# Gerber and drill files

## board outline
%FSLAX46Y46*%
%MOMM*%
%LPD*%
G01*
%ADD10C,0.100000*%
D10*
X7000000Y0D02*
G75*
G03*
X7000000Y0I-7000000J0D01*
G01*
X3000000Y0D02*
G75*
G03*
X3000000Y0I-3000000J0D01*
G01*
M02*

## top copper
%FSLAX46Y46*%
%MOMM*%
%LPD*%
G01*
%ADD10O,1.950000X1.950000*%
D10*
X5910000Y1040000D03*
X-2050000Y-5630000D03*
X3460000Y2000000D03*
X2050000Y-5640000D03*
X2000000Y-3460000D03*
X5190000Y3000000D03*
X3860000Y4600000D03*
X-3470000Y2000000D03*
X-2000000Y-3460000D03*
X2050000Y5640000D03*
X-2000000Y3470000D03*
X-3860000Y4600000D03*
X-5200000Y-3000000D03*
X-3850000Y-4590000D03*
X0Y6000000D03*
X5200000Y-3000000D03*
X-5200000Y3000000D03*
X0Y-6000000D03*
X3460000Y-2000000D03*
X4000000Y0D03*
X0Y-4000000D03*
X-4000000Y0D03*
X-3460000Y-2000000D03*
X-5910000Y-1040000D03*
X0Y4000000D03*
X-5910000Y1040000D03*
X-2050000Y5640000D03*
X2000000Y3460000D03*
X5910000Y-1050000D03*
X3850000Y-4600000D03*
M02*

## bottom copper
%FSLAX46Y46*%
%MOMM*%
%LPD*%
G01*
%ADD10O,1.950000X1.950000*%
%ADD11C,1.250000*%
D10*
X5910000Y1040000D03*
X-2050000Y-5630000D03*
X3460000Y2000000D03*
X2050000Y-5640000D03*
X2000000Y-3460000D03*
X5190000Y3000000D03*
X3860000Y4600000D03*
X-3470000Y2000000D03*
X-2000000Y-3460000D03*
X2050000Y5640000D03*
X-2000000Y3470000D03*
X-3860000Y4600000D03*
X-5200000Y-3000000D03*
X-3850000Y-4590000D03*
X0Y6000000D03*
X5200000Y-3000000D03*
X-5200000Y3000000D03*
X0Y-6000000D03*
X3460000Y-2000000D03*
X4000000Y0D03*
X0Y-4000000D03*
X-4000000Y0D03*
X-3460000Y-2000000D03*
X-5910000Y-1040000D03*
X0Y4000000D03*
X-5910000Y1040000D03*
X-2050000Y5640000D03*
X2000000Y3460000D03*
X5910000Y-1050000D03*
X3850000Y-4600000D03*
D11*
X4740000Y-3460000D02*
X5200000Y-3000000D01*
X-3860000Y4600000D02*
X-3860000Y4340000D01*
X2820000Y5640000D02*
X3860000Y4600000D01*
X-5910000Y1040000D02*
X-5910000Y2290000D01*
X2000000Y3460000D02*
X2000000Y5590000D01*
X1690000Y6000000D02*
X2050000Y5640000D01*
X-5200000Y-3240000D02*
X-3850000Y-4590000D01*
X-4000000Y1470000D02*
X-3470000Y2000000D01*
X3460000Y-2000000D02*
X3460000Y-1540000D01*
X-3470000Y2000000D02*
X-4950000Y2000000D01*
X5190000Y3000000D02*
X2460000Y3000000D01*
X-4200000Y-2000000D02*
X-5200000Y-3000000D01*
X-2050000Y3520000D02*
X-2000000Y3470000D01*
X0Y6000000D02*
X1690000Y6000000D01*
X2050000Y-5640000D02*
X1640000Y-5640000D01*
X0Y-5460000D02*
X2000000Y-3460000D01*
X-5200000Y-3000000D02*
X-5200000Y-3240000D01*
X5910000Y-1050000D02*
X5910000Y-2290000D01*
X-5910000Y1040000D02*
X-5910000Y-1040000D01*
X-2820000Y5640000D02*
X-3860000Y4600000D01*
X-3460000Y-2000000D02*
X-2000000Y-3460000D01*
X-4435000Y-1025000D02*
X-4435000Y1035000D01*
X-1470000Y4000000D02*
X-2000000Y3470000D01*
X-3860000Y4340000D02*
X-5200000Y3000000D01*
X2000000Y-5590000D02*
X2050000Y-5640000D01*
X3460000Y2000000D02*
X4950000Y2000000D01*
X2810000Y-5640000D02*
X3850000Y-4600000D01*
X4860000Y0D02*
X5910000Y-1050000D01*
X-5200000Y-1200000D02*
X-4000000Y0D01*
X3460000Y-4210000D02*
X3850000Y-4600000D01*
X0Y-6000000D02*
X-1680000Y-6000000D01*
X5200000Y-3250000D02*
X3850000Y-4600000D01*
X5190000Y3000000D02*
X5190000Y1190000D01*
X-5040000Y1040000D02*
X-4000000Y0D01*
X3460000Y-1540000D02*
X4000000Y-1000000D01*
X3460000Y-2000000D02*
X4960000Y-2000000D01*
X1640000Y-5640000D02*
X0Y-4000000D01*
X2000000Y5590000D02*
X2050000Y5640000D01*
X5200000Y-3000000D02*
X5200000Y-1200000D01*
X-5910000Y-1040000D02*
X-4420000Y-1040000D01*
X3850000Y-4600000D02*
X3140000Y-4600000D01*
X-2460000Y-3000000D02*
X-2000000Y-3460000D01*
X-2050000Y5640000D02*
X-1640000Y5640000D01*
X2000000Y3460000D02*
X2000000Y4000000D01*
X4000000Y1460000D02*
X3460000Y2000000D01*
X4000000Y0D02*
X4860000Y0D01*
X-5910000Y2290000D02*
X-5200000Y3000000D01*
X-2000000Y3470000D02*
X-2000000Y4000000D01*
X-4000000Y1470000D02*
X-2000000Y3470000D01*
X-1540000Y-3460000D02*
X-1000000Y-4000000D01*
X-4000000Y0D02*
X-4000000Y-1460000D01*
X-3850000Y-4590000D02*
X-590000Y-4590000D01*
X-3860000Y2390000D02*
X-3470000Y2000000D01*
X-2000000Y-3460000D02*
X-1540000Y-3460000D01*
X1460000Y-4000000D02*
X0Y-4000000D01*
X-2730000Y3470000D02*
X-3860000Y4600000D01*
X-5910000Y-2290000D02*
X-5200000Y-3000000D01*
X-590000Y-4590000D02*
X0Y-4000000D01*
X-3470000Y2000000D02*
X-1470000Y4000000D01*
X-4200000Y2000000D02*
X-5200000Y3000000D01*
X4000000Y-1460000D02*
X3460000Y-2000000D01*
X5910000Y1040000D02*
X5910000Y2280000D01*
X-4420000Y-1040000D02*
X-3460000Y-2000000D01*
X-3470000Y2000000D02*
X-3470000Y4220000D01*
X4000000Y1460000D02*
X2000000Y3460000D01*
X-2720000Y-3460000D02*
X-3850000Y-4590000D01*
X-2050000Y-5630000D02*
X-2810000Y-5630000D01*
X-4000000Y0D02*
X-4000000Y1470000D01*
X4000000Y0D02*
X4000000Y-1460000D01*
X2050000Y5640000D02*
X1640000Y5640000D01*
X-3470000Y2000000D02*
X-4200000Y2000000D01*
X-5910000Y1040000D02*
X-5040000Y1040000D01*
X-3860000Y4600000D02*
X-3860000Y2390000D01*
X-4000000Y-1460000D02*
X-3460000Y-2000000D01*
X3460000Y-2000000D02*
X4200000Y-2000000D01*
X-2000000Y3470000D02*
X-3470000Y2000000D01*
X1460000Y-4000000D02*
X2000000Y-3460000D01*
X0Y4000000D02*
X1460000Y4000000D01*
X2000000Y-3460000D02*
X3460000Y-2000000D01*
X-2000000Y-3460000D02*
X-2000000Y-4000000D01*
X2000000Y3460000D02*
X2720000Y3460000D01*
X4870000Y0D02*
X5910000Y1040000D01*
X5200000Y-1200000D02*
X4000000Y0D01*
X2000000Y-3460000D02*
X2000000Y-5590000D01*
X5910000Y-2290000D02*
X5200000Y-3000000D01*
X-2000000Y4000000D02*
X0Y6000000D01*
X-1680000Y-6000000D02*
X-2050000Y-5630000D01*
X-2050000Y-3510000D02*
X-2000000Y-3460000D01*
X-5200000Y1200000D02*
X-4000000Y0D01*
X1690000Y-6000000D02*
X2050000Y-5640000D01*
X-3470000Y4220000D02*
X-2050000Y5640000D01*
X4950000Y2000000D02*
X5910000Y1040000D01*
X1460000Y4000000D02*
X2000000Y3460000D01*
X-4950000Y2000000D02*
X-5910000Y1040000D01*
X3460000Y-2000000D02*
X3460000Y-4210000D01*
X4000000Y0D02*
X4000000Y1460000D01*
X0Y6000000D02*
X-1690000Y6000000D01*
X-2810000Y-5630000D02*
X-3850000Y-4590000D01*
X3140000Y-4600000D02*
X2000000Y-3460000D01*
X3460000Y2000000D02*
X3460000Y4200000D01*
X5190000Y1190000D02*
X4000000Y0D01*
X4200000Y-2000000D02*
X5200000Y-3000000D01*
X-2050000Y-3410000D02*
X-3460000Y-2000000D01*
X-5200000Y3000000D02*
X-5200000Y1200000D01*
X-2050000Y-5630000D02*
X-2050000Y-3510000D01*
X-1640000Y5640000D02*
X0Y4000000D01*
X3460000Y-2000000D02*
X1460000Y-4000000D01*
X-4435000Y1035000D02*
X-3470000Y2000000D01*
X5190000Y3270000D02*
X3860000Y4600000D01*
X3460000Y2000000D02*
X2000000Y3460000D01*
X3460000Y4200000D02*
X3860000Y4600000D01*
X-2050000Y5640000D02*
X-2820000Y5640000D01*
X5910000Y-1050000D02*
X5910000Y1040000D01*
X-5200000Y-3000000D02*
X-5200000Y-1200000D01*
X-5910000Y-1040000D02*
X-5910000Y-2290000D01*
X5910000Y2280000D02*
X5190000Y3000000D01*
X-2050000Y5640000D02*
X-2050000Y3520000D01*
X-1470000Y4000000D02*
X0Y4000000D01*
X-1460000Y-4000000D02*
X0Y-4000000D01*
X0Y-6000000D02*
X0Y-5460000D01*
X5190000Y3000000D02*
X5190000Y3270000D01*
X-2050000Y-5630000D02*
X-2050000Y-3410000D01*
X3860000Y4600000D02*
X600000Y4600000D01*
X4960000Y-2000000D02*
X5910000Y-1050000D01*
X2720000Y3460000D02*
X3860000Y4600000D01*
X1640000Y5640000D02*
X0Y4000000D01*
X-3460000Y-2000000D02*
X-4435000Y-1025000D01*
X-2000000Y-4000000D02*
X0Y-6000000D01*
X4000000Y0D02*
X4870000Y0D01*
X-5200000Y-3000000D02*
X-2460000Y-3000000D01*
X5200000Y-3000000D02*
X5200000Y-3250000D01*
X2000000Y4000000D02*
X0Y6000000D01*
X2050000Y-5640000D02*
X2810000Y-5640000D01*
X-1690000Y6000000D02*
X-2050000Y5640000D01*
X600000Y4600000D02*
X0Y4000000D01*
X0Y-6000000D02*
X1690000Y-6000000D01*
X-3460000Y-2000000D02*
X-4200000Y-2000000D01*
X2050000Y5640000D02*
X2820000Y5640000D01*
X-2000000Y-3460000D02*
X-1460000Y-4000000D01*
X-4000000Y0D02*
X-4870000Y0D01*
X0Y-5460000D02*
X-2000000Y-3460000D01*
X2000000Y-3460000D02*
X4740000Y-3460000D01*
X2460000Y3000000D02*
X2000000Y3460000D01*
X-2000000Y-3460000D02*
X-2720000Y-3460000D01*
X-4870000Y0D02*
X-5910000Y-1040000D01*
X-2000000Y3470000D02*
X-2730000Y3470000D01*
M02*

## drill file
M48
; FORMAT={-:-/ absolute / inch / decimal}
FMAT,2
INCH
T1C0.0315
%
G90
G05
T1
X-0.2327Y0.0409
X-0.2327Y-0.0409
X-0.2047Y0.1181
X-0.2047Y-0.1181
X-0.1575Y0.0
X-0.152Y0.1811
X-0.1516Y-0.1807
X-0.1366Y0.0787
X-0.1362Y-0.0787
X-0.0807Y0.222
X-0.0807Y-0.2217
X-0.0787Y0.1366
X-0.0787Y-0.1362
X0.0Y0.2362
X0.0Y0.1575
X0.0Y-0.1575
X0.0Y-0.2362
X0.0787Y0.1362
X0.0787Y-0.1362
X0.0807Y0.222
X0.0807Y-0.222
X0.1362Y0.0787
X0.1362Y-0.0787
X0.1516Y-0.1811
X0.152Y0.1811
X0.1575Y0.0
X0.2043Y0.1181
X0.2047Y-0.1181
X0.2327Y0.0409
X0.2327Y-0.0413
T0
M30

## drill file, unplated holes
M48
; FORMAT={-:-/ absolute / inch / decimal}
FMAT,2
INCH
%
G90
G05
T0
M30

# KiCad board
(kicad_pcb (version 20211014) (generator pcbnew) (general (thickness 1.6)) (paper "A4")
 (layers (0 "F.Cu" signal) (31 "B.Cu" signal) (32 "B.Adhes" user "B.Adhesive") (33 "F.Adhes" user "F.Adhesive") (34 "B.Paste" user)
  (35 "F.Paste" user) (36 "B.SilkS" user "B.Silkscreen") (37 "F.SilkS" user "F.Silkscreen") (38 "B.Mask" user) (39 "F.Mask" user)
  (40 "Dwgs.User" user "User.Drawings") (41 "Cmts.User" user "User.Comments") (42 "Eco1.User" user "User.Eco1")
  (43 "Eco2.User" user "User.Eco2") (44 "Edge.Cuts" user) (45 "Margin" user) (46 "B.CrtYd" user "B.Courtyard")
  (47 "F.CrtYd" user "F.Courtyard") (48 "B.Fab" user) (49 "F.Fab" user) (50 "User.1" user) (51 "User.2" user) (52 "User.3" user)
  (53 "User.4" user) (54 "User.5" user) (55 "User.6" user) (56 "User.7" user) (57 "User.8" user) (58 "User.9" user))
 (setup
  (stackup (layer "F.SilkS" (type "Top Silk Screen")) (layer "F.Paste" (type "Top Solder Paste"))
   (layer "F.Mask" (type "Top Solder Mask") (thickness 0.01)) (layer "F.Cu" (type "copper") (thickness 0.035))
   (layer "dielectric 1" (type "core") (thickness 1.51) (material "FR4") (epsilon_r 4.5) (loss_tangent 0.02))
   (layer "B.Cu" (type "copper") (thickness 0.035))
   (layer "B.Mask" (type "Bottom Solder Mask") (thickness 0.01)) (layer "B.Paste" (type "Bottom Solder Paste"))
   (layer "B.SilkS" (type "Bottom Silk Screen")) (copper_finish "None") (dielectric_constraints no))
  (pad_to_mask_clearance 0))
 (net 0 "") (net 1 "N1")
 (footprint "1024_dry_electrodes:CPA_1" (layer "F.Cu") (at 5.91 -1.04)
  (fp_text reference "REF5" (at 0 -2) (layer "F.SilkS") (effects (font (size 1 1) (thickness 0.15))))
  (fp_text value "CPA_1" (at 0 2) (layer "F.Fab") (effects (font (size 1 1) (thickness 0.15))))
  (pad "1" thru_hole oval (at 0 0) (size 1.95 1.95) (drill 0.8) (layers *.Cu *.Mask) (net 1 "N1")))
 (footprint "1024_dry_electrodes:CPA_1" (layer "F.Cu") (at -2.05 5.63)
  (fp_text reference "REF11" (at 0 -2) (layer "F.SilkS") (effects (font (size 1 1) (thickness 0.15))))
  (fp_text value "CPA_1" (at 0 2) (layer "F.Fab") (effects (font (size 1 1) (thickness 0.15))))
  (pad "1" thru_hole oval (at 0 0) (size 1.95 1.95) (drill 0.8) (layers *.Cu *.Mask) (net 1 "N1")))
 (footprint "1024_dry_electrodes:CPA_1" (layer "F.Cu") (at 3.46 -2)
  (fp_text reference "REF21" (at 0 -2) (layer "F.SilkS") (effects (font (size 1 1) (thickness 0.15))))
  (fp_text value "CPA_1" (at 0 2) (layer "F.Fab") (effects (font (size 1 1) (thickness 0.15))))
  (pad "1" thru_hole oval (at 0 0) (size 1.95 1.95) (drill 0.8) (layers *.Cu *.Mask) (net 1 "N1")))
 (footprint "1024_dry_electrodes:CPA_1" (layer "F.Cu") (at 2.05 5.64)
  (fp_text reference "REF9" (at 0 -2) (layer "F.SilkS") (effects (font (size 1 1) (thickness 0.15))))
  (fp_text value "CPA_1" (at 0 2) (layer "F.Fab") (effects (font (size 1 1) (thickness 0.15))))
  (pad "1" thru_hole oval (at 0 0) (size 1.95 1.95) (drill 0.8) (layers *.Cu *.Mask) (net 1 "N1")))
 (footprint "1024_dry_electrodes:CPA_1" (layer "F.Cu") (at 2 3.46)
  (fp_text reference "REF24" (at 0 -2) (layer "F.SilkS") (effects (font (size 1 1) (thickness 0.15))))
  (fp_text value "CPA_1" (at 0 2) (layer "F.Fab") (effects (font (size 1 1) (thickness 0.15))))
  (pad "1" thru_hole oval (at 0 0) (size 1.95 1.95) (drill 0.8) (layers *.Cu *.Mask) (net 1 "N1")))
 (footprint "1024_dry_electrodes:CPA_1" (layer "F.Cu") (at 5.19 -3)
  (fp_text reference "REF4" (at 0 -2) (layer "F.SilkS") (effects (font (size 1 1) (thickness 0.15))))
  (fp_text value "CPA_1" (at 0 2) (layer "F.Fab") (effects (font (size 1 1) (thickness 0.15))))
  (pad "1" thru_hole oval (at 0 0) (size 1.95 1.95) (drill 0.8) (layers *.Cu *.Mask) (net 1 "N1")))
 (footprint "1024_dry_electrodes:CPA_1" (layer "F.Cu") (at 3.86 -4.6)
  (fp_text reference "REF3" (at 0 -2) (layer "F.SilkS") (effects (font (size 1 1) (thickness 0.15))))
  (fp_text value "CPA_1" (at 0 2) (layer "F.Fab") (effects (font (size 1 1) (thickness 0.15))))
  (pad "1" thru_hole oval (at 0 0) (size 1.95 1.95) (drill 0.8) (layers *.Cu *.Mask) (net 1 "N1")))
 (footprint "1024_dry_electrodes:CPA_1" (layer "F.Cu") (at -3.47 -2)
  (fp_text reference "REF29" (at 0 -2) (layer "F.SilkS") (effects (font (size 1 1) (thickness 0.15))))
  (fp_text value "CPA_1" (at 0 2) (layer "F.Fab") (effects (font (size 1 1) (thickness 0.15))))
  (pad "1" thru_hole oval (at 0 0) (size 1.95 1.95) (drill 0.8) (layers *.Cu *.Mask) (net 1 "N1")))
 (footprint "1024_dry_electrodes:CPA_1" (layer "F.Cu") (at -2 3.46)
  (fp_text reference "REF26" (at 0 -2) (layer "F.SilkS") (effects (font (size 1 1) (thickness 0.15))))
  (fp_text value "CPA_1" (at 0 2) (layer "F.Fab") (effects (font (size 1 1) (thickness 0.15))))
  (pad "1" thru_hole oval (at 0 0) (size 1.95 1.95) (drill 0.8) (layers *.Cu *.Mask) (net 1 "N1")))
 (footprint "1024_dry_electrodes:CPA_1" (layer "F.Cu") (at 2.05 -5.64)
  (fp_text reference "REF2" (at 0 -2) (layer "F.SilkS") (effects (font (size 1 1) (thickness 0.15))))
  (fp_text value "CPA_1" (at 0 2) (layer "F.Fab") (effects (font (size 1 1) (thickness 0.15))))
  (pad "1" thru_hole oval (at 0 0) (size 1.95 1.95) (drill 0.8) (layers *.Cu *.Mask) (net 1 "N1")))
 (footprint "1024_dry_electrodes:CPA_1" (layer "F.Cu") (at -2 -3.47)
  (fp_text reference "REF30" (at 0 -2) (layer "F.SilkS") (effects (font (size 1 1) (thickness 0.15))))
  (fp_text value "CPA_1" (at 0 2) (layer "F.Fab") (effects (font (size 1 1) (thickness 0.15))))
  (pad "1" thru_hole oval (at 0 0) (size 1.95 1.95) (drill 0.8) (layers *.Cu *.Mask) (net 1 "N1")))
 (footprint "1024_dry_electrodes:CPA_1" (layer "F.Cu") (at -3.86 -4.6)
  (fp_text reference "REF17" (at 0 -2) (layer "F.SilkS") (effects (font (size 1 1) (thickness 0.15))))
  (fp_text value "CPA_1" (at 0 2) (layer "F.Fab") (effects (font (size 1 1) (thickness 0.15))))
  (pad "1" thru_hole oval (at 0 0) (size 1.95 1.95) (drill 0.8) (layers *.Cu *.Mask) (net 1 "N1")))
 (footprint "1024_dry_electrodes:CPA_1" (layer "F.Cu") (at -5.2 3)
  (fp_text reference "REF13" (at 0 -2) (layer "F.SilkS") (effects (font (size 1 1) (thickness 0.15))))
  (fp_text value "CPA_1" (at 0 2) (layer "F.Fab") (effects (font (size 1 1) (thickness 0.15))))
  (pad "1" thru_hole oval (at 0 0) (size 1.95 1.95) (drill 0.8) (layers *.Cu *.Mask) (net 1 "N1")))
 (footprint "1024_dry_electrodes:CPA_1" (layer "F.Cu") (at -3.85 4.59)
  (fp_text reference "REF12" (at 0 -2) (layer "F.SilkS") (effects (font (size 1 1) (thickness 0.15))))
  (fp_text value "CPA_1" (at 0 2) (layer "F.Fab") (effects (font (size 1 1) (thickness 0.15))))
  (pad "1" thru_hole oval (at 0 0) (size 1.95 1.95) (drill 0.8) (layers *.Cu *.Mask) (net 1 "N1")))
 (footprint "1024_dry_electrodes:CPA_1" (layer "F.Cu") (at 0 -6)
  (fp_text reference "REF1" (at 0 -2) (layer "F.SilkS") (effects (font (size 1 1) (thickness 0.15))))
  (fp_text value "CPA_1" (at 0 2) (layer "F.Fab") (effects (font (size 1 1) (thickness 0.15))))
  (pad "1" thru_hole oval (at 0 0) (size 1.95 1.95) (drill 0.8) (layers *.Cu *.Mask) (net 1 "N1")))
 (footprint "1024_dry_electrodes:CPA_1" (layer "F.Cu") (at 5.2 3)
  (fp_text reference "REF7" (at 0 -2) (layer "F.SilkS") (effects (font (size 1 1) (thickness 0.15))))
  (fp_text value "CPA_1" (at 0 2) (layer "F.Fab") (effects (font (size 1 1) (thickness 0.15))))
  (pad "1" thru_hole oval (at 0 0) (size 1.95 1.95) (drill 0.8) (layers *.Cu *.Mask) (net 1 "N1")))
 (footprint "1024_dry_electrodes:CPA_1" (layer "F.Cu") (at -5.2 -3)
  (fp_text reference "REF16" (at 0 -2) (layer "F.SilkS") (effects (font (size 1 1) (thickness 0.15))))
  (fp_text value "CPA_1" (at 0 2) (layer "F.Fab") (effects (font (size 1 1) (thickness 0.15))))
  (pad "1" thru_hole oval (at 0 0) (size 1.95 1.95) (drill 0.8) (layers *.Cu *.Mask) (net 1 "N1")))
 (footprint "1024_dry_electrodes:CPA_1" (layer "F.Cu") (at 0 6)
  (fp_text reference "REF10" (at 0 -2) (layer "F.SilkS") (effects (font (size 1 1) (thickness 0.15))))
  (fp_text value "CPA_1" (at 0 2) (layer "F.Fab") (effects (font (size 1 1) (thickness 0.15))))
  (pad "1" thru_hole oval (at 0 0) (size 1.95 1.95) (drill 0.8) (layers *.Cu *.Mask) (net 1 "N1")))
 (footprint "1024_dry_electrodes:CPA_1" (layer "F.Cu") (at 3.46 2)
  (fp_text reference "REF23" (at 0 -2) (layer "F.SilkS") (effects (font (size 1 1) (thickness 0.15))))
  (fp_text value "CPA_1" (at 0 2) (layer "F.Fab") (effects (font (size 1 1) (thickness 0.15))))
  (pad "1" thru_hole oval (at 0 0) (size 1.95 1.95) (drill 0.8) (layers *.Cu *.Mask) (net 1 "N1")))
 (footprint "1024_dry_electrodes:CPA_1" (layer "F.Cu") (at 4 0)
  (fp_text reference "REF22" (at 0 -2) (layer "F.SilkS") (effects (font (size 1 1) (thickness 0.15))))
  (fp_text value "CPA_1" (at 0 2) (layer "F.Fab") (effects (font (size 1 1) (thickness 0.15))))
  (pad "1" thru_hole oval (at 0 0) (size 1.95 1.95) (drill 0.8) (layers *.Cu *.Mask) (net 1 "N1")))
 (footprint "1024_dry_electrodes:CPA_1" (layer "F.Cu") (at 0 4)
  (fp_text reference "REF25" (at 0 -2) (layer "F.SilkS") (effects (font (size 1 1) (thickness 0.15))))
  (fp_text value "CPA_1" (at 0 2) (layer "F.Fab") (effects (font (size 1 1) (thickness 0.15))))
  (pad "1" thru_hole oval (at 0 0) (size 1.95 1.95) (drill 0.8) (layers *.Cu *.Mask) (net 1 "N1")))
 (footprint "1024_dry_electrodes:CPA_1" (layer "F.Cu") (at -4 0)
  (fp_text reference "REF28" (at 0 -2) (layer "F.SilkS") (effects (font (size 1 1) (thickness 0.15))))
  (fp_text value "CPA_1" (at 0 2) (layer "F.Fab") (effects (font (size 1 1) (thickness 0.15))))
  (pad "1" thru_hole oval (at 0 0) (size 1.95 1.95) (drill 0.8) (layers *.Cu *.Mask) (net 1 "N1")))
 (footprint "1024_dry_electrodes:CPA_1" (layer "F.Cu") (at -3.46 2)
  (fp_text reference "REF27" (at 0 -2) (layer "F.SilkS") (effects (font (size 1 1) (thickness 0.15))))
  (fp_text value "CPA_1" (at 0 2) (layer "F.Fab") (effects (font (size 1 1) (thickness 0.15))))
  (pad "1" thru_hole oval (at 0 0) (size 1.95 1.95) (drill 0.8) (layers *.Cu *.Mask) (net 1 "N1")))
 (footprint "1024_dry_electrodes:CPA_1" (layer "F.Cu") (at -5.91 1.04)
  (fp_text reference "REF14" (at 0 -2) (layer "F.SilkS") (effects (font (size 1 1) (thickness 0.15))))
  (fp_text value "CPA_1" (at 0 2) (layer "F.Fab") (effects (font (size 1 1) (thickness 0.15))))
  (pad "1" thru_hole oval (at 0 0) (size 1.95 1.95) (drill 0.8) (layers *.Cu *.Mask) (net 1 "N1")))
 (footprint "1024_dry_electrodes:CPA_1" (layer "F.Cu") (at 0 -4)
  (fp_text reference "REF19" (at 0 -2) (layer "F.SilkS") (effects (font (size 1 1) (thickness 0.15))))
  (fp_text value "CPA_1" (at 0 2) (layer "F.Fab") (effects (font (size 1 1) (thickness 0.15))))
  (pad "1" thru_hole oval (at 0 0) (size 1.95 1.95) (drill 0.8) (layers *.Cu *.Mask) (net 1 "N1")))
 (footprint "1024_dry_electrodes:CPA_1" (layer "F.Cu") (at -5.91 -1.04)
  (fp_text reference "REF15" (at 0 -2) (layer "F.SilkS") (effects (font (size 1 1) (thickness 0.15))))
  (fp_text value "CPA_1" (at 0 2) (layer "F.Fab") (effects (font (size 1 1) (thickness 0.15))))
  (pad "1" thru_hole oval (at 0 0) (size 1.95 1.95) (drill 0.8) (layers *.Cu *.Mask) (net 1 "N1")))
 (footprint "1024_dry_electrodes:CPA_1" (layer "F.Cu") (at -2.05 -5.64)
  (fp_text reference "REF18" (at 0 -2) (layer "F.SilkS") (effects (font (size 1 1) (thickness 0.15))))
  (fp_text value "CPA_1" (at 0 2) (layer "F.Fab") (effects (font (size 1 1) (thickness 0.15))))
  (pad "1" thru_hole oval (at 0 0) (size 1.95 1.95) (drill 0.8) (layers *.Cu *.Mask) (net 1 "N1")))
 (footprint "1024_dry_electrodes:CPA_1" (layer "F.Cu") (at 2 -3.46)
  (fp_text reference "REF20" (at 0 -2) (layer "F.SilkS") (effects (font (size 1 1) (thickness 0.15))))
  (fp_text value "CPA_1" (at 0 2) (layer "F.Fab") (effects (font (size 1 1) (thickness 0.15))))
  (pad "1" thru_hole oval (at 0 0) (size 1.95 1.95) (drill 0.8) (layers *.Cu *.Mask) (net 1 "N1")))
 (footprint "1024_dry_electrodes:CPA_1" (layer "F.Cu") (at 5.91 1.05)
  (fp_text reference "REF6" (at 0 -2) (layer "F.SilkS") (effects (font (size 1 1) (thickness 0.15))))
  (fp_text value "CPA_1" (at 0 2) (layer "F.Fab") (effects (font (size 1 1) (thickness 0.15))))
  (pad "1" thru_hole oval (at 0 0) (size 1.95 1.95) (drill 0.8) (layers *.Cu *.Mask) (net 1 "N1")))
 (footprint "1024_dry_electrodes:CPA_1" (layer "F.Cu") (at 3.85 4.6)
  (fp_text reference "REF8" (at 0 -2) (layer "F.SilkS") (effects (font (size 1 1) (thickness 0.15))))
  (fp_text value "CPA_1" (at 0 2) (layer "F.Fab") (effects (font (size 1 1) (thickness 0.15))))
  (pad "1" thru_hole oval (at 0 0) (size 1.95 1.95) (drill 0.8) (layers *.Cu *.Mask) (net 1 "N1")))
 (gr_circle (center 0 0) (end 7 0) (layer "Edge.Cuts") (width 0.1) (fill none))
 (gr_circle (center 0 0) (end 3 0) (layer "Edge.Cuts") (width 0.1) (fill none))
 (segment (start 4.74 3.46) (end 5.2 3) (width 1.25) (layer "B.Cu") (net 1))
 (segment (start -3.86 -4.6) (end -3.86 -4.34) (width 1.25) (layer "B.Cu") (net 1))
 (segment (start 2.82 -5.64) (end 3.86 -4.6) (width 1.25) (layer "B.Cu") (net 1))
 (segment (start -5.91 -1.04) (end -5.91 -2.29) (width 1.25) (layer "B.Cu") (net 1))
 (segment (start 2 -3.46) (end 2 -5.59) (width 1.25) (layer "B.Cu") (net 1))
 (segment (start 1.69 -6) (end 2.05 -5.64) (width 1.25) (layer "B.Cu") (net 1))
 (segment (start -5.2 3.24) (end -3.85 4.59) (width 1.25) (layer "B.Cu") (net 1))
 (segment (start -4 -1.47) (end -3.47 -2) (width 1.25) (layer "B.Cu") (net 1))
 (segment (start 3.46 2) (end 3.46 1.54) (width 1.25) (layer "B.Cu") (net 1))
 (segment (start -3.47 -2) (end -4.95 -2) (width 1.25) (layer "B.Cu") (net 1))
 (segment (start 5.19 -3) (end 2.46 -3) (width 1.25) (layer "B.Cu") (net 1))
 (segment (start -4.2 2) (end -5.2 3) (width 1.25) (layer "B.Cu") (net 1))
 (segment (start -2.05 -3.52) (end -2 -3.47) (width 1.25) (layer "B.Cu") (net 1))
 (segment (start 0 -6) (end 1.69 -6) (width 1.25) (layer "B.Cu") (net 1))
 (segment (start 2.05 5.64) (end 1.64 5.64) (width 1.25) (layer "B.Cu") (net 1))
 (segment (start 0 5.46) (end 2 3.46) (width 1.25) (layer "B.Cu") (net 1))
 (segment (start -5.2 3) (end -5.2 3.24) (width 1.25) (layer "B.Cu") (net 1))
 (segment (start 5.91 1.05) (end 5.91 2.29) (width 1.25) (layer "B.Cu") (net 1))
 (segment (start -5.91 -1.04) (end -5.91 1.04) (width 1.25) (layer "B.Cu") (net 1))
 (segment (start -2.82 -5.64) (end -3.86 -4.6) (width 1.25) (layer "B.Cu") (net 1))
 (segment (start -3.46 2) (end -2 3.46) (width 1.25) (layer "B.Cu") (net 1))
 (segment (start -4.435 1.025) (end -4.435 -1.035) (width 1.25) (layer "B.Cu") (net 1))
 (segment (start -1.47 -4) (end -2 -3.47) (width 1.25) (layer "B.Cu") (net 1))
 (segment (start -3.86 -4.34) (end -5.2 -3) (width 1.25) (layer "B.Cu") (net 1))
 (segment (start 2 5.59) (end 2.05 5.64) (width 1.25) (layer "B.Cu") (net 1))
 (segment (start 3.46 -2) (end 4.95 -2) (width 1.25) (layer "B.Cu") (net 1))
 (segment (start 2.81 5.64) (end 3.85 4.6) (width 1.25) (layer "B.Cu") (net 1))
 (segment (start 4.86 0) (end 5.91 1.05) (width 1.25) (layer "B.Cu") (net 1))
 (segment (start -5.2 1.2) (end -4 0) (width 1.25) (layer "B.Cu") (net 1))
 (segment (start 3.46 4.21) (end 3.85 4.6) (width 1.25) (layer "B.Cu") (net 1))
 (segment (start 0 6) (end -1.68 6) (width 1.25) (layer "B.Cu") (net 1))
 (segment (start 5.2 3.25) (end 3.85 4.6) (width 1.25) (layer "B.Cu") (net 1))
 (segment (start 5.19 -3) (end 5.19 -1.19) (width 1.25) (layer "B.Cu") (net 1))
 (segment (start -5.04 -1.04) (end -4 0) (width 1.25) (layer "B.Cu") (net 1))
 (segment (start 3.46 1.54) (end 4 1) (width 1.25) (layer "B.Cu") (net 1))
 (segment (start 3.46 2) (end 4.96 2) (width 1.25) (layer "B.Cu") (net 1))
 (segment (start 1.64 5.64) (end 0 4) (width 1.25) (layer "B.Cu") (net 1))
 (segment (start 2 -5.59) (end 2.05 -5.64) (width 1.25) (layer "B.Cu") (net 1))
 (segment (start 5.2 3) (end 5.2 1.2) (width 1.25) (layer "B.Cu") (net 1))
 (segment (start -5.91 1.04) (end -4.42 1.04) (width 1.25) (layer "B.Cu") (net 1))
 (segment (start 3.85 4.6) (end 3.14 4.6) (width 1.25) (layer "B.Cu") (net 1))
 (segment (start -2.46 3) (end -2 3.46) (width 1.25) (layer "B.Cu") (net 1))
 (segment (start -2.05 -5.64) (end -1.64 -5.64) (width 1.25) (layer "B.Cu") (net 1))
 (segment (start 2 -3.46) (end 2 -4) (width 1.25) (layer "B.Cu") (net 1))
 (segment (start 4 -1.46) (end 3.46 -2) (width 1.25) (layer "B.Cu") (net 1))
 (segment (start 4 0) (end 4.86 0) (width 1.25) (layer "B.Cu") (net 1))
 (segment (start -5.91 -2.29) (end -5.2 -3) (width 1.25) (layer "B.Cu") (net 1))
 (segment (start -2 -3.47) (end -2 -4) (width 1.25) (layer "B.Cu") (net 1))
 (segment (start -4 -1.47) (end -2 -3.47) (width 1.25) (layer "B.Cu") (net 1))
 (segment (start -1.54 3.46) (end -1 4) (width 1.25) (layer "B.Cu") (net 1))
 (segment (start -4 0) (end -4 1.46) (width 1.25) (layer "B.Cu") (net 1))
 (segment (start -3.85 4.59) (end -0.59 4.59) (width 1.25) (layer "B.Cu") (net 1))
 (segment (start -3.86 -2.39) (end -3.47 -2) (width 1.25) (layer "B.Cu") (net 1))
 (segment (start -2 3.46) (end -1.54 3.46) (width 1.25) (layer "B.Cu") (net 1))
 (segment (start 1.46 4) (end 0 4) (width 1.25) (layer "B.Cu") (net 1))
 (segment (start -2.73 -3.47) (end -3.86 -4.6) (width 1.25) (layer "B.Cu") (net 1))
 (segment (start -5.91 2.29) (end -5.2 3) (width 1.25) (layer "B.Cu") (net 1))
 (segment (start -0.59 4.59) (end 0 4) (width 1.25) (layer "B.Cu") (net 1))
 (segment (start -3.47 -2) (end -1.47 -4) (width 1.25) (layer "B.Cu") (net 1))
 (segment (start -4.2 -2) (end -5.2 -3) (width 1.25) (layer "B.Cu") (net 1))
 (segment (start 4 1.46) (end 3.46 2) (width 1.25) (layer "B.Cu") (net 1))
 (segment (start 5.91 -1.04) (end 5.91 -2.28) (width 1.25) (layer "B.Cu") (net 1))
 (segment (start -4.42 1.04) (end -3.46 2) (width 1.25) (layer "B.Cu") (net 1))
 (segment (start -3.47 -2) (end -3.47 -4.22) (width 1.25) (layer "B.Cu") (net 1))
 (segment (start 4 -1.46) (end 2 -3.46) (width 1.25) (layer "B.Cu") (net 1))
 (segment (start -2.72 3.46) (end -3.85 4.59) (width 1.25) (layer "B.Cu") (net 1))
 (segment (start -2.05 5.63) (end -2.81 5.63) (width 1.25) (layer "B.Cu") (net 1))
 (segment (start -4 0) (end -4 -1.47) (width 1.25) (layer "B.Cu") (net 1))
 (segment (start 4 0) (end 4 1.46) (width 1.25) (layer "B.Cu") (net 1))
 (segment (start 2.05 -5.64) (end 1.64 -5.64) (width 1.25) (layer "B.Cu") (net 1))
 (segment (start -3.47 -2) (end -4.2 -2) (width 1.25) (layer "B.Cu") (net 1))
 (segment (start -5.91 -1.04) (end -5.04 -1.04) (width 1.25) (layer "B.Cu") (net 1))
 (segment (start -3.86 -4.6) (end -3.86 -2.39) (width 1.25) (layer "B.Cu") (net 1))
 (segment (start -4 1.46) (end -3.46 2) (width 1.25) (layer "B.Cu") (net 1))
 (segment (start 3.46 2) (end 4.2 2) (width 1.25) (layer "B.Cu") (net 1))
 (segment (start -2 -3.47) (end -3.47 -2) (width 1.25) (layer "B.Cu") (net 1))
 (segment (start 1.46 4) (end 2 3.46) (width 1.25) (layer "B.Cu") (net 1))
 (segment (start 0 -4) (end 1.46 -4) (width 1.25) (layer "B.Cu") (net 1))
 (segment (start 2 3.46) (end 3.46 2) (width 1.25) (layer "B.Cu") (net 1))
 (segment (start -2 3.46) (end -2 4) (width 1.25) (layer "B.Cu") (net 1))
 (segment (start 2 -3.46) (end 2.72 -3.46) (width 1.25) (layer "B.Cu") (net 1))
 (segment (start 4.87 0) (end 5.91 -1.04) (width 1.25) (layer "B.Cu") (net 1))
 (segment (start 5.2 1.2) (end 4 0) (width 1.25) (layer "B.Cu") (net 1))
 (segment (start 2 3.46) (end 2 5.59) (width 1.25) (layer "B.Cu") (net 1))
 (segment (start 5.91 2.29) (end 5.2 3) (width 1.25) (layer "B.Cu") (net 1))
 (segment (start -2 -4) (end 0 -6) (width 1.25) (layer "B.Cu") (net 1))
 (segment (start -1.68 6) (end -2.05 5.63) (width 1.25) (layer "B.Cu") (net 1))
 (segment (start -2.05 3.51) (end -2 3.46) (width 1.25) (layer "B.Cu") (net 1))
 (segment (start -5.2 -1.2) (end -4 0) (width 1.25) (layer "B.Cu") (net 1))
 (segment (start 1.69 6) (end 2.05 5.64) (width 1.25) (layer "B.Cu") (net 1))
 (segment (start -3.47 -4.22) (end -2.05 -5.64) (width 1.25) (layer "B.Cu") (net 1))
 (segment (start 4.95 -2) (end 5.91 -1.04) (width 1.25) (layer "B.Cu") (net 1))
 (segment (start 1.46 -4) (end 2 -3.46) (width 1.25) (layer "B.Cu") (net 1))
 (segment (start -4.95 -2) (end -5.91 -1.04) (width 1.25) (layer "B.Cu") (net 1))
 (segment (start 3.46 2) (end 3.46 4.21) (width 1.25) (layer "B.Cu") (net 1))
 (segment (start 4 0) (end 4 -1.46) (width 1.25) (layer "B.Cu") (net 1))
 (segment (start 0 -6) (end -1.69 -6) (width 1.25) (layer "B.Cu") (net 1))
 (segment (start -2.81 5.63) (end -3.85 4.59) (width 1.25) (layer "B.Cu") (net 1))
 (segment (start 3.14 4.6) (end 2 3.46) (width 1.25) (layer "B.Cu") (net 1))
 (segment (start 3.46 -2) (end 3.46 -4.2) (width 1.25) (layer "B.Cu") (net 1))
 (segment (start 5.19 -1.19) (end 4 0) (width 1.25) (layer "B.Cu") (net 1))
 (segment (start 4.2 2) (end 5.2 3) (width 1.25) (layer "B.Cu") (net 1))
 (segment (start -2.05 3.41) (end -3.46 2) (width 1.25) (layer "B.Cu") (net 1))
 (segment (start -5.2 -3) (end -5.2 -1.2) (width 1.25) (layer "B.Cu") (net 1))
 (segment (start -2.05 5.63) (end -2.05 3.51) (width 1.25) (layer "B.Cu") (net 1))
 (segment (start -1.64 -5.64) (end 0 -4) (width 1.25) (layer "B.Cu") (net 1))
 (segment (start 3.46 2) (end 1.46 4) (width 1.25) (layer "B.Cu") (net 1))
 (segment (start -4.435 -1.035) (end -3.47 -2) (width 1.25) (layer "B.Cu") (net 1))
 (segment (start 5.19 -3.27) (end 3.86 -4.6) (width 1.25) (layer "B.Cu") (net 1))
 (segment (start 3.46 -2) (end 2 -3.46) (width 1.25) (layer "B.Cu") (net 1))
 (segment (start 3.46 -4.2) (end 3.86 -4.6) (width 1.25) (layer "B.Cu") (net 1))
 (segment (start -2.05 -5.64) (end -2.82 -5.64) (width 1.25) (layer "B.Cu") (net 1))
 (segment (start 5.91 1.05) (end 5.91 -1.04) (width 1.25) (layer "B.Cu") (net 1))
 (segment (start -5.2 3) (end -5.2 1.2) (width 1.25) (layer "B.Cu") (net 1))
 (segment (start -5.91 1.04) (end -5.91 2.29) (width 1.25) (layer "B.Cu") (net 1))
 (segment (start 5.91 -2.28) (end 5.19 -3) (width 1.25) (layer "B.Cu") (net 1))
 (segment (start -2.05 -5.64) (end -2.05 -3.52) (width 1.25) (layer "B.Cu") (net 1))
 (segment (start -1.47 -4) (end 0 -4) (width 1.25) (layer "B.Cu") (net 1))
 (segment (start -1.46 4) (end 0 4) (width 1.25) (layer "B.Cu") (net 1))
 (segment (start 0 6) (end 0 5.46) (width 1.25) (layer "B.Cu") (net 1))
 (segment (start 5.19 -3) (end 5.19 -3.27) (width 1.25) (layer "B.Cu") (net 1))
 (segment (start -2.05 5.63) (end -2.05 3.41) (width 1.25) (layer "B.Cu") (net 1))
 (segment (start 3.86 -4.6) (end 0.6 -4.6) (width 1.25) (layer "B.Cu") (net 1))
 (segment (start 4.96 2) (end 5.91 1.05) (width 1.25) (layer "B.Cu") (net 1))
 (segment (start 2.72 -3.46) (end 3.86 -4.6) (width 1.25) (layer "B.Cu") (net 1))
 (segment (start 1.64 -5.64) (end 0 -4) (width 1.25) (layer "B.Cu") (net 1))
 (segment (start -3.46 2) (end -4.435 1.025) (width 1.25) (layer "B.Cu") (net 1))
 (segment (start -2 4) (end 0 6) (width 1.25) (layer "B.Cu") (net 1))
 (segment (start 4 0) (end 4.87 0) (width 1.25) (layer "B.Cu") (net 1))
 (segment (start -5.2 3) (end -2.46 3) (width 1.25) (layer "B.Cu") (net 1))
 (segment (start 5.2 3) (end 5.2 3.25) (width 1.25) (layer "B.Cu") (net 1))
 (segment (start 2 -4) (end 0 -6) (width 1.25) (layer "B.Cu") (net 1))
 (segment (start 2.05 5.64) (end 2.81 5.64) (width 1.25) (layer "B.Cu") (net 1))
 (segment (start -1.69 -6) (end -2.05 -5.64) (width 1.25) (layer "B.Cu") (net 1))
 (segment (start 0.6 -4.6) (end 0 -4) (width 1.25) (layer "B.Cu") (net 1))
 (segment (start 0 6) (end 1.69 6) (width 1.25) (layer "B.Cu") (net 1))
 (segment (start -3.46 2) (end -4.2 2) (width 1.25) (layer "B.Cu") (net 1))
 (segment (start 2.05 -5.64) (end 2.82 -5.64) (width 1.25) (layer "B.Cu") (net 1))
 (segment (start -2 3.46) (end -1.46 4) (width 1.25) (layer "B.Cu") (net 1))
 (segment (start -4 0) (end -4.87 0) (width 1.25) (layer "B.Cu") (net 1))
 (segment (start 0 5.46) (end -2 3.46) (width 1.25) (layer "B.Cu") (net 1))
 (segment (start 2 3.46) (end 4.74 3.46) (width 1.25) (layer "B.Cu") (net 1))
 (segment (start 2.46 -3) (end 2 -3.46) (width 1.25) (layer "B.Cu") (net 1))
 (segment (start -2 3.46) (end -2.72 3.46) (width 1.25) (layer "B.Cu") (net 1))
 (segment (start -4.87 0) (end -5.91 1.04) (width 1.25) (layer "B.Cu") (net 1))
 (segment (start -2 -3.47) (end -2.73 -3.47) (width 1.25) (layer "B.Cu") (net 1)))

